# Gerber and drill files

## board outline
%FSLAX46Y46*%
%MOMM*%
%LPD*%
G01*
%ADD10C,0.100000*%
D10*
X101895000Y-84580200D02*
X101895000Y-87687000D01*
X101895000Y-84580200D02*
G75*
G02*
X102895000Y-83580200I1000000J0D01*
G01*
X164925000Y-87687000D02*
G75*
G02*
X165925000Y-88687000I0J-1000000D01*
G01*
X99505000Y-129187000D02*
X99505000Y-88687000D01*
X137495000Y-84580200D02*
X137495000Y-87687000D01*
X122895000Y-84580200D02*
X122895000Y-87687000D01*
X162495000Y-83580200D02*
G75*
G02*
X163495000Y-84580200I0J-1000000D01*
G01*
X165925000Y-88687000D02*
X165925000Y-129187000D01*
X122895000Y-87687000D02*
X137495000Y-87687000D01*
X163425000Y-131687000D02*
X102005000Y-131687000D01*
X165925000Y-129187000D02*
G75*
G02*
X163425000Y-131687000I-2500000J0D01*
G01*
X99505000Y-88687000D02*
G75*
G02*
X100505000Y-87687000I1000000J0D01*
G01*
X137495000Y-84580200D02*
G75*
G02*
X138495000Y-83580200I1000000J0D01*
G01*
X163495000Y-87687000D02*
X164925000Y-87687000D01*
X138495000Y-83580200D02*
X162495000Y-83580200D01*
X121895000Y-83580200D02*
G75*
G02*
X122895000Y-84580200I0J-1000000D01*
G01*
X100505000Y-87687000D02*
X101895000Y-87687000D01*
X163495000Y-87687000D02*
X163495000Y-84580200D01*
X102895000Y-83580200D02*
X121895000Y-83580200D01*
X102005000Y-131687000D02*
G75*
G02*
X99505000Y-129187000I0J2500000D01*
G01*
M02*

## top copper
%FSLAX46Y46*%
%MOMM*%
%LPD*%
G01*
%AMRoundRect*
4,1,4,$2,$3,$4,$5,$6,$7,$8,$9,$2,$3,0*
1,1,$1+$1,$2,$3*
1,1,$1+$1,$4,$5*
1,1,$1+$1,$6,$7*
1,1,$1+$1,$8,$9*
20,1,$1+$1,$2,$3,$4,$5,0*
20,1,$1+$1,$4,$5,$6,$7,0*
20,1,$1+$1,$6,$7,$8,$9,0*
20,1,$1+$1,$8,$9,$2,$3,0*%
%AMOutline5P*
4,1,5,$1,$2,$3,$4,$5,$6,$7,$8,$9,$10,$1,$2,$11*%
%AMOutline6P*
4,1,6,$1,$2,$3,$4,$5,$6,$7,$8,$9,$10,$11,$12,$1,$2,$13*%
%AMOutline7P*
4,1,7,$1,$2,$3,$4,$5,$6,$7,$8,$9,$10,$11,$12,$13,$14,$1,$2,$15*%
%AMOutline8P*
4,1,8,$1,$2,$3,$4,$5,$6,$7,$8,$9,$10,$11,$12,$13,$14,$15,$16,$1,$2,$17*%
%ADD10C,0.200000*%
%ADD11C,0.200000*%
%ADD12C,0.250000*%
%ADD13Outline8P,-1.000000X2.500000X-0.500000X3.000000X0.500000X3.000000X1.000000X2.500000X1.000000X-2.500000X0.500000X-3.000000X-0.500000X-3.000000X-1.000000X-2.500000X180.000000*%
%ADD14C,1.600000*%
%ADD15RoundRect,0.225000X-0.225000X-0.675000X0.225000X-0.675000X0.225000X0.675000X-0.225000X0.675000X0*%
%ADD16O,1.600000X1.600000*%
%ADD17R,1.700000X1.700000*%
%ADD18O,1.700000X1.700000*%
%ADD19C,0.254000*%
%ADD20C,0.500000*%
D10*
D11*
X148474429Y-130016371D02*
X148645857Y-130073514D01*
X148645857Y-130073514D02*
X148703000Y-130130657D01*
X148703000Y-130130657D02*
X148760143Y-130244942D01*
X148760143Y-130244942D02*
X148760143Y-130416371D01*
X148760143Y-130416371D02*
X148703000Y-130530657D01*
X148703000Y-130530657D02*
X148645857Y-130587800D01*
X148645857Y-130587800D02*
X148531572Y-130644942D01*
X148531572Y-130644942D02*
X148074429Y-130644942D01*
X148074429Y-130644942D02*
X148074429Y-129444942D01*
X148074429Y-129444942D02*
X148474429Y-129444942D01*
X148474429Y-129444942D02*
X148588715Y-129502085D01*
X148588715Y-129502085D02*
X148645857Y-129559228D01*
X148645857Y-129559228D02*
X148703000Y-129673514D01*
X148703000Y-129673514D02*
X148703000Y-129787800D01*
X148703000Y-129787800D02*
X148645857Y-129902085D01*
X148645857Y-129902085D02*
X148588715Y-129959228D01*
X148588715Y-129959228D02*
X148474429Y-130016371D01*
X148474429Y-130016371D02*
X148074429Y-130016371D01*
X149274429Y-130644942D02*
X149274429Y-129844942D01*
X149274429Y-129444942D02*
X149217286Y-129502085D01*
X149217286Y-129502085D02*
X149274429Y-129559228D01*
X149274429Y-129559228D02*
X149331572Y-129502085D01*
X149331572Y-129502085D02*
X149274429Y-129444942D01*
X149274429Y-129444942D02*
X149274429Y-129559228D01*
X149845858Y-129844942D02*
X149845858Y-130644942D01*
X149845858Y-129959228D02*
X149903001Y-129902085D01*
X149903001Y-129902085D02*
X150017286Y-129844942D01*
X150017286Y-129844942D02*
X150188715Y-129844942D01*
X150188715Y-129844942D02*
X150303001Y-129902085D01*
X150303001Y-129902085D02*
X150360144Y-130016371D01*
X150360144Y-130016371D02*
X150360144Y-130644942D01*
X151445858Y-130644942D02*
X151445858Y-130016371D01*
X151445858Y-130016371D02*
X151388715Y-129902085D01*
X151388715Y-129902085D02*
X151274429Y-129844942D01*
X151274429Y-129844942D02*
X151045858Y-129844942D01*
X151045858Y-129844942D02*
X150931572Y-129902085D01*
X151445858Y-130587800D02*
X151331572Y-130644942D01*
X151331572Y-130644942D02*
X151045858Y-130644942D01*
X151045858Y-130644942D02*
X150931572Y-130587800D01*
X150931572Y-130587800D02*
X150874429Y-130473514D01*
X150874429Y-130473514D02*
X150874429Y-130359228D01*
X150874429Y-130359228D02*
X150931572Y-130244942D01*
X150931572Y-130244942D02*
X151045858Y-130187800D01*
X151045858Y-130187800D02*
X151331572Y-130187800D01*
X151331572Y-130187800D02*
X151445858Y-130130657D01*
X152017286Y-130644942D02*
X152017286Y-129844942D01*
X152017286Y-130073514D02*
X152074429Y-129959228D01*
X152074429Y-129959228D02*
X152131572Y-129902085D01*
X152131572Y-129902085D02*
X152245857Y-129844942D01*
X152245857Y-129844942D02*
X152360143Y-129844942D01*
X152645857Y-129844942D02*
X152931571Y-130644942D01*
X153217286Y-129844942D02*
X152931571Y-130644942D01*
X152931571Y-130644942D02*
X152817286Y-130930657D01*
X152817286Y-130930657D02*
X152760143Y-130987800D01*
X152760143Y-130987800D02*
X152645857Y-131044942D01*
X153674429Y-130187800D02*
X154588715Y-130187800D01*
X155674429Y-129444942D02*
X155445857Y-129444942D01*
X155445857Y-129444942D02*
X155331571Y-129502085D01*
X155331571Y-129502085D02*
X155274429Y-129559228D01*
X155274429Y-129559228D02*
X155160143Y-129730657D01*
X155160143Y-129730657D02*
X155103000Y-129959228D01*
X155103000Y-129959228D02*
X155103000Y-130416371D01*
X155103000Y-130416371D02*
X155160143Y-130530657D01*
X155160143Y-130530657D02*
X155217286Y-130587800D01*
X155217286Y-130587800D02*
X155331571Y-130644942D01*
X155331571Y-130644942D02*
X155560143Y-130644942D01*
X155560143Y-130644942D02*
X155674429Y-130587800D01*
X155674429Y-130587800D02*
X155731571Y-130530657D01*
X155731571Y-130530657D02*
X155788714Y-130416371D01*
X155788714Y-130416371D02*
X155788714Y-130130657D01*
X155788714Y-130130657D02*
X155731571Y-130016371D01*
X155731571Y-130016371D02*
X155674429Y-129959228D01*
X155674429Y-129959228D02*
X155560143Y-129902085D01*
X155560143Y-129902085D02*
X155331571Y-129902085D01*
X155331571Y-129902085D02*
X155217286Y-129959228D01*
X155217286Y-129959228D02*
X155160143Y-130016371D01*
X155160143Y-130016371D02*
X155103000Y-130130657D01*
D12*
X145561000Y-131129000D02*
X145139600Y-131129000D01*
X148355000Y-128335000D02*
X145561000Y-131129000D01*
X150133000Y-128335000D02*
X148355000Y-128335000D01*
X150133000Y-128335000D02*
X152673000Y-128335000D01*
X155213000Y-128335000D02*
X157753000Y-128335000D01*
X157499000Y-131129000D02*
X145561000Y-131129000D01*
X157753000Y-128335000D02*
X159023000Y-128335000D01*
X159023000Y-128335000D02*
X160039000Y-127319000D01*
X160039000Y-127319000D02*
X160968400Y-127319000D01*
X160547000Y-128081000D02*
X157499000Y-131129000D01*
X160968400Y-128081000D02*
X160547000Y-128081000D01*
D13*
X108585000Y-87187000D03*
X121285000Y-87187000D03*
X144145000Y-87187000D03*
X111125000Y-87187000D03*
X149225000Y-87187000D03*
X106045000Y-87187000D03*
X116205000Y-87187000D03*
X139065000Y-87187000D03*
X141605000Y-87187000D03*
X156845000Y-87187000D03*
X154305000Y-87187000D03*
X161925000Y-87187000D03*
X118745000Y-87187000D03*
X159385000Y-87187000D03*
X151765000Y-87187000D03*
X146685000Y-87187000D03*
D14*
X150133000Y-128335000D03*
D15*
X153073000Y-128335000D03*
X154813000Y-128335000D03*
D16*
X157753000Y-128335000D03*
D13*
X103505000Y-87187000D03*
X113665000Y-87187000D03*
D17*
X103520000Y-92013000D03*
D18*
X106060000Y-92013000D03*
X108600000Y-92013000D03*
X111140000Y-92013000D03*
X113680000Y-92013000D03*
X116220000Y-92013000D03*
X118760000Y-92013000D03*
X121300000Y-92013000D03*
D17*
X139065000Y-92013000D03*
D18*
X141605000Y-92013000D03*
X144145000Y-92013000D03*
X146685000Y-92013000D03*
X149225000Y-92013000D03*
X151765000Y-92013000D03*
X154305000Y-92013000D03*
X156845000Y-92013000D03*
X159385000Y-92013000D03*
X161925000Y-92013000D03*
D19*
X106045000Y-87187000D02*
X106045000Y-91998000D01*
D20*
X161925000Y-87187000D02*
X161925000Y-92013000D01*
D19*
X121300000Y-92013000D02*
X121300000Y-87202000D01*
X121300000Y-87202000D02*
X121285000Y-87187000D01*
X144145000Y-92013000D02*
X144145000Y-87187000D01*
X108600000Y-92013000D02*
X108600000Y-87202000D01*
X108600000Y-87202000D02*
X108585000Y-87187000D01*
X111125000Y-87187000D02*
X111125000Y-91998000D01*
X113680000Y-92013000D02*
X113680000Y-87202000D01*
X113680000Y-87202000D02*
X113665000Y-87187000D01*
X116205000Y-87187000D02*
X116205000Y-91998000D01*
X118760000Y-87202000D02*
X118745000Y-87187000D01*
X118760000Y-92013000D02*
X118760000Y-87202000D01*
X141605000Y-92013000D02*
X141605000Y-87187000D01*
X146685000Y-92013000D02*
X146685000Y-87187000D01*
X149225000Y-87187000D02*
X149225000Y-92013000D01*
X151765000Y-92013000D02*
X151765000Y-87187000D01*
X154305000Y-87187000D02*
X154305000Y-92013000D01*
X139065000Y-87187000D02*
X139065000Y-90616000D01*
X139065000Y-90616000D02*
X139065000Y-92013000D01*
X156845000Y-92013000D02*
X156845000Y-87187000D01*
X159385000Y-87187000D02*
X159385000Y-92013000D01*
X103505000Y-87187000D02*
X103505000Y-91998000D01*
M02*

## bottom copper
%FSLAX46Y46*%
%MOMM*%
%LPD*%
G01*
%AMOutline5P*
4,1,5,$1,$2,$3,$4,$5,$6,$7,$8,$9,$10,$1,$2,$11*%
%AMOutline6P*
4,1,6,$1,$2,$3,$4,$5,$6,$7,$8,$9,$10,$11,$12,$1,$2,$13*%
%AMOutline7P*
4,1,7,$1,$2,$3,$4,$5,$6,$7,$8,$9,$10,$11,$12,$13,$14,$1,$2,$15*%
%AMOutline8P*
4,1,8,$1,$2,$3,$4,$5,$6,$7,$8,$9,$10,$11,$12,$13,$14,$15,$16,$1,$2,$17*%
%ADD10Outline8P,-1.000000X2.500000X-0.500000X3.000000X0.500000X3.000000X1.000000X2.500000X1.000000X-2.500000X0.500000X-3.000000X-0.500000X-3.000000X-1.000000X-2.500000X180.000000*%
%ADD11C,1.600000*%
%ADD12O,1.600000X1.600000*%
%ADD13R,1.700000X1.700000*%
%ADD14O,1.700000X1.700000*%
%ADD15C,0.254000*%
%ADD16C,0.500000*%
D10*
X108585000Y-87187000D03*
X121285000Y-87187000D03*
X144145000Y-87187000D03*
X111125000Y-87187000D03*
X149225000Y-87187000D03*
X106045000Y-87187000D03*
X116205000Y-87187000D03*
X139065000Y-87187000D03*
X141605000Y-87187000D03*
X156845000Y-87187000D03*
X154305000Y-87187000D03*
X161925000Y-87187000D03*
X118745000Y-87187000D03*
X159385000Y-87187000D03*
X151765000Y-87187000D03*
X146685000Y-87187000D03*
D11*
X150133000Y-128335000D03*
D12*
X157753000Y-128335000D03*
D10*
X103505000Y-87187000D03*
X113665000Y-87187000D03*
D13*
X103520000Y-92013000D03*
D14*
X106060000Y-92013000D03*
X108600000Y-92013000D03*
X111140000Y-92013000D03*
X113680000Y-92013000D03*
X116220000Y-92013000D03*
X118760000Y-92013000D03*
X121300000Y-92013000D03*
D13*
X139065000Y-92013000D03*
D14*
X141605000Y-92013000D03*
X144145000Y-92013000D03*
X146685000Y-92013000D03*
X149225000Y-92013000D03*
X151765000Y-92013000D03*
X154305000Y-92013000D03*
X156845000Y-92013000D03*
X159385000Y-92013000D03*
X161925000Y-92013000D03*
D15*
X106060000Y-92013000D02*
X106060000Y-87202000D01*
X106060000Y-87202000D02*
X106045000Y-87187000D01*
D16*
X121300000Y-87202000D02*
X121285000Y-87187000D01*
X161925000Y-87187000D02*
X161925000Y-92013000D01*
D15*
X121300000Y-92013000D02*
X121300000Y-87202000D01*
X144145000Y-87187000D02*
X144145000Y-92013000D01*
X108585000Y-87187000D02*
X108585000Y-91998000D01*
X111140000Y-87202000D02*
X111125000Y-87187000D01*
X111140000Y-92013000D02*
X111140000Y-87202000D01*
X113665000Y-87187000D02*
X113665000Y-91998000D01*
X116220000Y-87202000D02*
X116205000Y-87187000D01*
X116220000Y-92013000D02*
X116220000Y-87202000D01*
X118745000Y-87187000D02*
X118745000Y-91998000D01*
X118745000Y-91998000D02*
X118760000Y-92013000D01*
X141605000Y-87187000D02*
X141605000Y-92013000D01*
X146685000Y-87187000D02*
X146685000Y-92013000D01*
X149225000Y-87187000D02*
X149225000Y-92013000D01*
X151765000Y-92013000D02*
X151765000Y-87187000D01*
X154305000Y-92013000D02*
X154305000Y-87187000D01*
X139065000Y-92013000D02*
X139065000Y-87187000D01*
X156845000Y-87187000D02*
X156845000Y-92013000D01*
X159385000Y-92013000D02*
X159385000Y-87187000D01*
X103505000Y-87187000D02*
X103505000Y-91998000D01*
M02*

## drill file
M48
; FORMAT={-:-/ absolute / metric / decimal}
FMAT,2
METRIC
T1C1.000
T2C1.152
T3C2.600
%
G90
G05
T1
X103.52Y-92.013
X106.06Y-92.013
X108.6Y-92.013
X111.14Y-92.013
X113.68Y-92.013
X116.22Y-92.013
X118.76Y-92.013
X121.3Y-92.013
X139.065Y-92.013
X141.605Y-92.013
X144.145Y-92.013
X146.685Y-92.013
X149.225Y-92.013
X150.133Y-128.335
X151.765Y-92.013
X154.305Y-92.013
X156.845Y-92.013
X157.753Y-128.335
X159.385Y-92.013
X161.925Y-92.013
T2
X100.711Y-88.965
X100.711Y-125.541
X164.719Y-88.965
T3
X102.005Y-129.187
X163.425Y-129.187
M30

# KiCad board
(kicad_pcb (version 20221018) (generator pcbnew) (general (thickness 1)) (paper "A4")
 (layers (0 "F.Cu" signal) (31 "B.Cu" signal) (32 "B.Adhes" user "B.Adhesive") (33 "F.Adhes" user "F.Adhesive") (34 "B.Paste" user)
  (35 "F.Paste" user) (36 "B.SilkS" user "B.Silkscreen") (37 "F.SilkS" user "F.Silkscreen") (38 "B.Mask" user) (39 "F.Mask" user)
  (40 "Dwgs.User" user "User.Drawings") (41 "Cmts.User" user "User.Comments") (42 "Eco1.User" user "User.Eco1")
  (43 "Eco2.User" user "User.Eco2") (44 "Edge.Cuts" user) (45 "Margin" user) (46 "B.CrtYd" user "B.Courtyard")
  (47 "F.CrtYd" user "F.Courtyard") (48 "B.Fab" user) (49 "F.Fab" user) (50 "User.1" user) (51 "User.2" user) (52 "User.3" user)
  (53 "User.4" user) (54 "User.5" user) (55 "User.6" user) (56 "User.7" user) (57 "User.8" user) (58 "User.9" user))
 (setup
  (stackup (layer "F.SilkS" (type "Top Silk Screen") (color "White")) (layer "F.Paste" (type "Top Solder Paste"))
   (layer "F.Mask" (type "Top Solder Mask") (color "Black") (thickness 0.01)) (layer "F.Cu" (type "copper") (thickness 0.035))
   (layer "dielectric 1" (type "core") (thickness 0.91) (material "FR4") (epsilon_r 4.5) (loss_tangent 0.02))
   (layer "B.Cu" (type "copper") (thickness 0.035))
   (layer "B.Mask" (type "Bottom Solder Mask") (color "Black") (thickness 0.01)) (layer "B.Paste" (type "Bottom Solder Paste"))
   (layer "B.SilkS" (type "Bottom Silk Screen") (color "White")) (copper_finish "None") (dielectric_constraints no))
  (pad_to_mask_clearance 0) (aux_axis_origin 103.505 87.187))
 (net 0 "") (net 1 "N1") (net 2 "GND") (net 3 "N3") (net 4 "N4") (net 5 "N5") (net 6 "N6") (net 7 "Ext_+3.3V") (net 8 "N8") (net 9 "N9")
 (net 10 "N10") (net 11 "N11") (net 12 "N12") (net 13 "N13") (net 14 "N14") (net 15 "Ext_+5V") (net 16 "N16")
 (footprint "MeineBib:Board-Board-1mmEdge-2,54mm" (layer "F.Cu") (at 108.585 87.187)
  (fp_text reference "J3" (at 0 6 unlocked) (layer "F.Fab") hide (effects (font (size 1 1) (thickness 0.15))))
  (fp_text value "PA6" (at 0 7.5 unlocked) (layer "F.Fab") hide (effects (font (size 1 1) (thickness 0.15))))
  (pad "1" smd roundrect (at 0 0 180) (size 2 6) (layers "F.Cu" "F.Paste" "F.Mask") (roundrect_rratio 0) (chamfer_ratio 0.25)
   (chamfer top_left top_right bottom_left bottom_right) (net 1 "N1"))
  (pad "1" smd roundrect (at 0 0 180) (size 2 6) (layers "B.Cu" "B.Paste" "B.Mask") (roundrect_rratio 0) (chamfer_ratio 0.25)
   (chamfer top_left top_right bottom_left bottom_right) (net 1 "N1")))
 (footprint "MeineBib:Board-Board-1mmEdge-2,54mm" (layer "F.Cu") (at 121.285 87.187)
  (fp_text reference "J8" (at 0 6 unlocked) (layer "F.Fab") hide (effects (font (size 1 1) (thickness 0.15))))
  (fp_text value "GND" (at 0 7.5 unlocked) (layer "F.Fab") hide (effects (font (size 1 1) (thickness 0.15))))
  (pad "1" smd roundrect (at 0 0 180) (size 2 6) (layers "F.Cu" "F.Paste" "F.Mask") (roundrect_rratio 0) (chamfer_ratio 0.25)
   (chamfer top_left top_right bottom_left bottom_right) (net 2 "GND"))
  (pad "1" smd roundrect (at 0 0 180) (size 2 6) (layers "B.Cu" "B.Paste" "B.Mask") (roundrect_rratio 0) (chamfer_ratio 0.25)
   (chamfer top_left top_right bottom_left bottom_right) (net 2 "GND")))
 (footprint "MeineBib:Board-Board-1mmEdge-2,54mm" (layer "F.Cu") (at 144.145 87.187)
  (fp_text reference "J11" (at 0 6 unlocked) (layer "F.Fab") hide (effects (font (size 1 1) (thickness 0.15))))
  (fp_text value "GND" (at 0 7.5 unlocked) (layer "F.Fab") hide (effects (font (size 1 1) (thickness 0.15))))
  (pad "1" smd roundrect (at 0 0 180) (size 2 6) (layers "F.Cu" "F.Paste" "F.Mask") (roundrect_rratio 0) (chamfer_ratio 0.25)
   (chamfer top_left top_right bottom_left bottom_right) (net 2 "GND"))
  (pad "1" smd roundrect (at 0 0 180) (size 2 6) (layers "B.Cu" "B.Paste" "B.Mask") (roundrect_rratio 0) (chamfer_ratio 0.25)
   (chamfer top_left top_right bottom_left bottom_right) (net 2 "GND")))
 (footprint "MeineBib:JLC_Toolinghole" (layer "F.Cu") (at 164.719 88.965)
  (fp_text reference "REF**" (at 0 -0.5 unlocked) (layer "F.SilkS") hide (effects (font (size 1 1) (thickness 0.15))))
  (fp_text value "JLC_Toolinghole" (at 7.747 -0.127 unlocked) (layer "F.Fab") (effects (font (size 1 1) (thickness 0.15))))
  (pad "" np_thru_hole circle (at 0 0) (size 1.3 1.3) (drill 1.152) (layers "*.Mask")))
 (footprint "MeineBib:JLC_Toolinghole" (layer "F.Cu") (at 100.711 125.541)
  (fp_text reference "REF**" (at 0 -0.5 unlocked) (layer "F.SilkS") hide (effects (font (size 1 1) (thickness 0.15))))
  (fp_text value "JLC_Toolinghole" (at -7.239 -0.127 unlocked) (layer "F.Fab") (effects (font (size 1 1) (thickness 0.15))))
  (pad "" np_thru_hole circle (at 0 0) (size 1.3 1.3) (drill 1.152) (layers "*.Mask")))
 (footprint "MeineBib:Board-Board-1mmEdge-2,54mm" (layer "F.Cu") (at 111.125 87.187)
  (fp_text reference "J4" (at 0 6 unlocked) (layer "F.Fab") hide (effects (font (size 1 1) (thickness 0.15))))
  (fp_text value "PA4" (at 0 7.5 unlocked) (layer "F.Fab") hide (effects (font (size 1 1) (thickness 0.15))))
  (pad "1" smd roundrect (at 0 0 180) (size 2 6) (layers "F.Cu" "F.Paste" "F.Mask") (roundrect_rratio 0) (chamfer_ratio 0.25)
   (chamfer top_left top_right bottom_left bottom_right) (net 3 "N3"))
  (pad "1" smd roundrect (at 0 0 180) (size 2 6) (layers "B.Cu" "B.Paste" "B.Mask") (roundrect_rratio 0) (chamfer_ratio 0.25)
   (chamfer top_left top_right bottom_left bottom_right) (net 3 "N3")))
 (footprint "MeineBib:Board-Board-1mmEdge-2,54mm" (layer "F.Cu") (at 149.225 87.187)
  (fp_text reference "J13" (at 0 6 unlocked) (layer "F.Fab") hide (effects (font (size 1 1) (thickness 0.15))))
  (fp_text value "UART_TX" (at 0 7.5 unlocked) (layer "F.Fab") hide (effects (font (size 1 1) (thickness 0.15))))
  (pad "1" smd roundrect (at 0 0 180) (size 2 6) (layers "F.Cu" "F.Paste" "F.Mask") (roundrect_rratio 0) (chamfer_ratio 0.25)
   (chamfer top_left top_right bottom_left bottom_right) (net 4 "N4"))
  (pad "1" smd roundrect (at 0 0 180) (size 2 6) (layers "B.Cu" "B.Paste" "B.Mask") (roundrect_rratio 0) (chamfer_ratio 0.25)
   (chamfer top_left top_right bottom_left bottom_right) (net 4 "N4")))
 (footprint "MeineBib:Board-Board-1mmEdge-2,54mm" (layer "F.Cu") (at 106.045 87.187)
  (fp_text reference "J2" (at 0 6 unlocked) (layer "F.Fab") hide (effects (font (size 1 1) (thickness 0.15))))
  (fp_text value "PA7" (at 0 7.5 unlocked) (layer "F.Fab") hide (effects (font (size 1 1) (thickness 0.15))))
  (pad "1" smd roundrect (at 0 0 180) (size 2 6) (layers "F.Cu" "F.Paste" "F.Mask") (roundrect_rratio 0) (chamfer_ratio 0.25)
   (chamfer top_left top_right bottom_left bottom_right) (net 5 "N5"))
  (pad "1" smd roundrect (at 0 0 180) (size 2 6) (layers "B.Cu" "B.Paste" "B.Mask") (roundrect_rratio 0) (chamfer_ratio 0.25)
   (chamfer top_left top_right bottom_left bottom_right) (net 5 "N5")))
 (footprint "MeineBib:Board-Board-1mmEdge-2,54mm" (layer "F.Cu") (at 116.205 87.187)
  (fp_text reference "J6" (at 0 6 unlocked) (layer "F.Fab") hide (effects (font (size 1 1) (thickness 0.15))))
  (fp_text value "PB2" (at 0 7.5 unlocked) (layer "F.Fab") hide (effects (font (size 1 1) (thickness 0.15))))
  (pad "1" smd roundrect (at 0 0 180) (size 2 6) (layers "F.Cu" "F.Paste" "F.Mask") (roundrect_rratio 0) (chamfer_ratio 0.25)
   (chamfer top_left top_right bottom_left bottom_right) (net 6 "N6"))
  (pad "1" smd roundrect (at 0 0 180) (size 2 6) (layers "B.Cu" "B.Paste" "B.Mask") (roundrect_rratio 0) (chamfer_ratio 0.25)
   (chamfer top_left top_right bottom_left bottom_right) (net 6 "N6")))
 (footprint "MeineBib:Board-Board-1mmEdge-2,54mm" (layer "F.Cu") (at 139.065 87.187)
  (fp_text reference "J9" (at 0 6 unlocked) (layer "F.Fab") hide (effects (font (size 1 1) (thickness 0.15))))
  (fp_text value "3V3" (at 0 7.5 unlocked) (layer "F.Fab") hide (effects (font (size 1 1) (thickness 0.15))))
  (pad "1" smd roundrect (at 0 0 180) (size 2 6) (layers "F.Cu" "F.Paste" "F.Mask") (roundrect_rratio 0) (chamfer_ratio 0.25)
   (chamfer top_left top_right bottom_left bottom_right) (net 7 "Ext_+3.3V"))
  (pad "1" smd roundrect (at 0 0 180) (size 2 6) (layers "B.Cu" "B.Paste" "B.Mask") (roundrect_rratio 0) (chamfer_ratio 0.25)
   (chamfer top_left top_right bottom_left bottom_right) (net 7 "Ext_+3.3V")))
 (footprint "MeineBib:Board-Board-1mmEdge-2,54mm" (layer "F.Cu") (at 141.605 87.187)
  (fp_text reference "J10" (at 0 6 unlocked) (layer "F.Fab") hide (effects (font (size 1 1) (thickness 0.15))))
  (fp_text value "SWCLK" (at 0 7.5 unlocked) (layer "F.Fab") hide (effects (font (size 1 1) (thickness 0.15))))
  (pad "1" smd roundrect (at 0 0 180) (size 2 6) (layers "F.Cu" "F.Paste" "F.Mask") (roundrect_rratio 0) (chamfer_ratio 0.25)
   (chamfer top_left top_right bottom_left bottom_right) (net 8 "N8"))
  (pad "1" smd roundrect (at 0 0 180) (size 2 6) (layers "B.Cu" "B.Paste" "B.Mask") (roundrect_rratio 0) (chamfer_ratio 0.25)
   (chamfer top_left top_right bottom_left bottom_right) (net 8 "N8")))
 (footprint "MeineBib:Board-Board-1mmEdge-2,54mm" (layer "F.Cu") (at 156.845 87.187)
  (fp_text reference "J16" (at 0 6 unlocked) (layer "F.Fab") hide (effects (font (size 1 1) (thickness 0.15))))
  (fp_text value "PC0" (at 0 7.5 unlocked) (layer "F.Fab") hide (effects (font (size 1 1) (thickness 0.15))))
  (pad "1" smd roundrect (at 0 0 180) (size 2 6) (layers "F.Cu" "F.Paste" "F.Mask") (roundrect_rratio 0) (chamfer_ratio 0.25)
   (chamfer top_left top_right bottom_left bottom_right) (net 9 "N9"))
  (pad "1" smd roundrect (at 0 0 180) (size 2 6) (layers "B.Cu" "B.Paste" "B.Mask") (roundrect_rratio 0) (chamfer_ratio 0.25)
   (chamfer top_left top_right bottom_left bottom_right) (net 9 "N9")))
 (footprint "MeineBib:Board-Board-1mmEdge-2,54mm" (layer "F.Cu") (at 154.305 87.187)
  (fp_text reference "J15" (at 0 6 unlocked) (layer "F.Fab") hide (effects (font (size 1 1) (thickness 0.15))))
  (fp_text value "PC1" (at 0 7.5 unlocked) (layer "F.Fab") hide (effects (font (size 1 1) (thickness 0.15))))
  (pad "1" smd roundrect (at 0 0 180) (size 2 6) (layers "F.Cu" "F.Paste" "F.Mask") (roundrect_rratio 0) (chamfer_ratio 0.25)
   (chamfer top_left top_right bottom_left bottom_right) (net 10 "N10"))
  (pad "1" smd roundrect (at 0 0 180) (size 2 6) (layers "B.Cu" "B.Paste" "B.Mask") (roundrect_rratio 0) (chamfer_ratio 0.25)
   (chamfer top_left top_right bottom_left bottom_right) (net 10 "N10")))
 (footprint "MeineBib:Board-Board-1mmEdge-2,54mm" (layer "F.Cu") (at 161.925 87.187)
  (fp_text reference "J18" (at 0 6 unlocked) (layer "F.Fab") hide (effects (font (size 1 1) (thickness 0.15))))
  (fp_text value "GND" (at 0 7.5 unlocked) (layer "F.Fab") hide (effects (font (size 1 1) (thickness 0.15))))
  (pad "1" smd roundrect (at 0 0 180) (size 2 6) (layers "F.Cu" "F.Paste" "F.Mask") (roundrect_rratio 0) (chamfer_ratio 0.25)
   (chamfer top_left top_right bottom_left bottom_right) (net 2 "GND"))
  (pad "1" smd roundrect (at 0 0 180) (size 2 6) (layers "B.Cu" "B.Paste" "B.Mask") (roundrect_rratio 0) (chamfer_ratio 0.25)
   (chamfer top_left top_right bottom_left bottom_right) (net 2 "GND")))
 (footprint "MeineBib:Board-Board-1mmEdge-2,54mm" (layer "F.Cu") (at 118.745 87.187)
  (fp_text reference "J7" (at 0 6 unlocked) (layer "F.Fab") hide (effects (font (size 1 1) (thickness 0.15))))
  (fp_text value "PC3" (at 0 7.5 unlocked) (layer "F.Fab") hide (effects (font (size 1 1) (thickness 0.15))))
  (pad "1" smd roundrect (at 0 0 180) (size 2 6) (layers "F.Cu" "F.Paste" "F.Mask") (roundrect_rratio 0) (chamfer_ratio 0.25)
   (chamfer top_left top_right bottom_left bottom_right) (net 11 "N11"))
  (pad "1" smd roundrect (at 0 0 180) (size 2 6) (layers "B.Cu" "B.Paste" "B.Mask") (roundrect_rratio 0) (chamfer_ratio 0.25)
   (chamfer top_left top_right bottom_left bottom_right) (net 11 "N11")))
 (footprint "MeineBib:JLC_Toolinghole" (layer "F.Cu") (at 100.711 88.965)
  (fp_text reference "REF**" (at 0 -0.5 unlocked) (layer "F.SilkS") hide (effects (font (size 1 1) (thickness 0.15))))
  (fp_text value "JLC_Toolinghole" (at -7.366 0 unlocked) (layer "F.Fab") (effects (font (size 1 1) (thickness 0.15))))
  (pad "" np_thru_hole circle (at 0 0) (size 1.3 1.3) (drill 1.152) (layers "*.Mask")))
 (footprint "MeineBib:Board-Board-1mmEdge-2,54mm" (layer "F.Cu") (at 159.385 87.187)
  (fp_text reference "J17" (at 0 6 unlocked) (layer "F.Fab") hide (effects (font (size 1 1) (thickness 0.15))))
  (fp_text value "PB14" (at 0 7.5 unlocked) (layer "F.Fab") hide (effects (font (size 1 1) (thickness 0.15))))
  (pad "1" smd roundrect (at 0 0 180) (size 2 6) (layers "F.Cu" "F.Paste" "F.Mask") (roundrect_rratio 0) (chamfer_ratio 0.25)
   (chamfer top_left top_right bottom_left bottom_right) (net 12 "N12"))
  (pad "1" smd roundrect (at 0 0 180) (size 2 6) (layers "B.Cu" "B.Paste" "B.Mask") (roundrect_rratio 0) (chamfer_ratio 0.25)
   (chamfer top_left top_right bottom_left bottom_right) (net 12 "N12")))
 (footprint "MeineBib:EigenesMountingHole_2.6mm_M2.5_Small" (layer "F.Cu") (at 102.005 129.187)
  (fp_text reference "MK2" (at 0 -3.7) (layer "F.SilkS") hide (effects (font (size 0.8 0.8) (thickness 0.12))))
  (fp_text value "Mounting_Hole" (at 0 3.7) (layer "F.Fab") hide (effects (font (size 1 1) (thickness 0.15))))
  (pad "" np_thru_hole circle (at 0 0) (size 2.6 2.6) (drill 2.6) (layers "F&B.Cu" "*.Mask") (solder_mask_margin 1.25) (clearance 1.25)))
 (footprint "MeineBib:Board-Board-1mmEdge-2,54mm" (layer "F.Cu") (at 151.765 87.187)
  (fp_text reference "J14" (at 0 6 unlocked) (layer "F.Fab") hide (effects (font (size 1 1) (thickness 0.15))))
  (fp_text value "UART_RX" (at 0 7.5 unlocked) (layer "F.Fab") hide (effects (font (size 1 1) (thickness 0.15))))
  (pad "1" smd roundrect (at 0 0 180) (size 2 6) (layers "F.Cu" "F.Paste" "F.Mask") (roundrect_rratio 0) (chamfer_ratio 0.25)
   (chamfer top_left top_right bottom_left bottom_right) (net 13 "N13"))
  (pad "1" smd roundrect (at 0 0 180) (size 2 6) (layers "B.Cu" "B.Paste" "B.Mask") (roundrect_rratio 0) (chamfer_ratio 0.25)
   (chamfer top_left top_right bottom_left bottom_right) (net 13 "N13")))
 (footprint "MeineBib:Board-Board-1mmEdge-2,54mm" (layer "F.Cu") (at 146.685 87.187)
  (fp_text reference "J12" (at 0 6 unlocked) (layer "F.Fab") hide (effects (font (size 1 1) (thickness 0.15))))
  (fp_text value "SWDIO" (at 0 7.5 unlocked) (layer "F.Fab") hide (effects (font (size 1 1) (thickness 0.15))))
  (pad "1" smd roundrect (at 0 0 180) (size 2 6) (layers "F.Cu" "F.Paste" "F.Mask") (roundrect_rratio 0) (chamfer_ratio 0.25)
   (chamfer top_left top_right bottom_left bottom_right) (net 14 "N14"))
  (pad "1" smd roundrect (at 0 0 180) (size 2 6) (layers "B.Cu" "B.Paste" "B.Mask") (roundrect_rratio 0) (chamfer_ratio 0.25)
   (chamfer top_left top_right bottom_left bottom_right) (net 14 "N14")))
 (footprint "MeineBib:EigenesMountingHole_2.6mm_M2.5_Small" (layer "F.Cu") (at 163.425 129.187)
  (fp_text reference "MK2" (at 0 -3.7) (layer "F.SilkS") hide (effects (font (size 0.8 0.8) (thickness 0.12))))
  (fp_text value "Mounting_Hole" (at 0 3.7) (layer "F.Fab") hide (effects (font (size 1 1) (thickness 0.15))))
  (pad "" np_thru_hole circle (at 0 0) (size 2.6 2.6) (drill 2.6) (layers "F&B.Cu" "*.Mask") (solder_mask_margin 1.25) (clearance 1.25)))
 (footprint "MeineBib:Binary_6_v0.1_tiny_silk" (layer "F.Cu") (at 153.9684 129.3002) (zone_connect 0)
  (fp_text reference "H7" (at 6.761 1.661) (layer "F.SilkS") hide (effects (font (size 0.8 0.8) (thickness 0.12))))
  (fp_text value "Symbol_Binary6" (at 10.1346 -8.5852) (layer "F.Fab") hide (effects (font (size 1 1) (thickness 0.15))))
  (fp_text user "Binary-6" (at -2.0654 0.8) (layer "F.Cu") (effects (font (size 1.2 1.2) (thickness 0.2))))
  (fp_line (start -8.4074 1.8288) (end -8.8288 1.8288) (stroke (width 0.25) (type solid)) (layer "F.Cu"))
  (fp_line (start -5.6134 -0.9652) (end -8.4074 1.8288) (stroke (width 0.25) (type solid)) (layer "F.Cu"))
  (fp_line (start -3.8354 -0.9652) (end -5.6134 -0.9652) (stroke (width 0.25) (type solid)) (layer "F.Cu"))
  (fp_line (start -3.8354 -0.9652) (end -1.2954 -0.9652) (stroke (width 0.25) (type solid)) (layer "F.Cu"))
  (fp_line (start 1.2446 -0.9652) (end 3.7846 -0.9652) (stroke (width 0.25) (type solid)) (layer "F.Cu"))
  (fp_line (start 3.5306 1.8288) (end -8.4074 1.8288) (stroke (width 0.25) (type solid)) (layer "F.Cu"))
  (fp_line (start 3.7846 -0.9652) (end 5.0546 -0.9652) (stroke (width 0.25) (type solid)) (layer "F.Cu"))
  (fp_line (start 5.0546 -0.9652) (end 6.0706 -1.9812) (stroke (width 0.25) (type solid)) (layer "F.Cu"))
  (fp_line (start 6.0706 -1.9812) (end 7 -1.9812) (stroke (width 0.25) (type solid)) (layer "F.Cu"))
  (fp_line (start 6.5786 -1.2192) (end 3.5306 1.8288) (stroke (width 0.25) (type solid)) (layer "F.Cu"))
  (fp_line (start 7 -1.2192) (end 6.5786 -1.2192) (stroke (width 0.25) (type solid)) (layer "F.Cu"))
  (pad "" thru_hole circle (at -3.8354 -0.9652) (size 1.6 1.6) (drill 1) (layers "*.Cu" "*.Mask") (zone_connect 0))
  (pad "" smd roundrect (at -0.8954 -0.9652) (size 0.9 1.8) (layers "F.Cu" "F.Mask") (roundrect_rratio 0.25) (zone_connect 0))
  (pad "" smd roundrect (at 0.8446 -0.9652) (size 0.9 1.8) (layers "F.Cu" "F.Mask") (roundrect_rratio 0.25) (zone_connect 0))
  (pad "" thru_hole oval (at 3.7846 -0.9652) (size 1.6 1.6) (drill 1) (layers "*.Cu" "*.Mask") (zone_connect 0)))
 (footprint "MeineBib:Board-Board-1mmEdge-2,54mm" (layer "F.Cu") (at 103.505 87.187)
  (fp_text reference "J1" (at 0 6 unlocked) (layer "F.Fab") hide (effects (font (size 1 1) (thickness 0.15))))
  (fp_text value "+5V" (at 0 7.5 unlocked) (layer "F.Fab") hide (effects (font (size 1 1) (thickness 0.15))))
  (pad "1" smd roundrect (at 0 0 180) (size 2 6) (layers "F.Cu" "F.Paste" "F.Mask") (roundrect_rratio 0) (chamfer_ratio 0.25)
   (chamfer top_left top_right bottom_left bottom_right) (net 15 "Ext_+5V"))
  (pad "1" smd roundrect (at 0 0 180) (size 2 6) (layers "B.Cu" "B.Paste" "B.Mask") (roundrect_rratio 0) (chamfer_ratio 0.25)
   (chamfer top_left top_right bottom_left bottom_right) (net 15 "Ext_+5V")))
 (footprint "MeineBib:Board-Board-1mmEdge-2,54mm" (layer "F.Cu") (at 113.665 87.187)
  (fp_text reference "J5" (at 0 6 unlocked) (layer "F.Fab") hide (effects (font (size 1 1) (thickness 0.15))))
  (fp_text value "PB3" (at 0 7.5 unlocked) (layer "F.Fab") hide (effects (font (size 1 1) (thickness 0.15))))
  (pad "1" smd roundrect (at 0 0 180) (size 2 6) (layers "F.Cu" "F.Paste" "F.Mask") (roundrect_rratio 0) (chamfer_ratio 0.25)
   (chamfer top_left top_right bottom_left bottom_right) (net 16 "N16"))
  (pad "1" smd roundrect (at 0 0 180) (size 2 6) (layers "B.Cu" "B.Paste" "B.Mask") (roundrect_rratio 0) (chamfer_ratio 0.25)
   (chamfer top_left top_right bottom_left bottom_right) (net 16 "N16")))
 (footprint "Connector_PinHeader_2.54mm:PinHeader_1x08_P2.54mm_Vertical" (layer "B.Cu") (at 103.52 92.013 -90)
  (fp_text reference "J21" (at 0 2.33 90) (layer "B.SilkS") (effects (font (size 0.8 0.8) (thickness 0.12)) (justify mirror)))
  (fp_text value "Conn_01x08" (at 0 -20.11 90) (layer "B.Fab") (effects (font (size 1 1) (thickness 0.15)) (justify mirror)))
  (pad "1" thru_hole rect (at 0 0 270) (size 1.7 1.7) (drill 1) (layers "*.Cu" "*.Mask") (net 15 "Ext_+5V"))
  (pad "2" thru_hole oval (at 0 -2.54 270) (size 1.7 1.7) (drill 1) (layers "*.Cu" "*.Mask") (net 5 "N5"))
  (pad "3" thru_hole oval (at 0 -5.08 270) (size 1.7 1.7) (drill 1) (layers "*.Cu" "*.Mask") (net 1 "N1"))
  (pad "4" thru_hole oval (at 0 -7.62 270) (size 1.7 1.7) (drill 1) (layers "*.Cu" "*.Mask") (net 3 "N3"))
  (pad "5" thru_hole oval (at 0 -10.16 270) (size 1.7 1.7) (drill 1) (layers "*.Cu" "*.Mask") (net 16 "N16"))
  (pad "6" thru_hole oval (at 0 -12.7 270) (size 1.7 1.7) (drill 1) (layers "*.Cu" "*.Mask") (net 6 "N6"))
  (pad "7" thru_hole oval (at 0 -15.24 270) (size 1.7 1.7) (drill 1) (layers "*.Cu" "*.Mask") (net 11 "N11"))
  (pad "8" thru_hole oval (at 0 -17.78 270) (size 1.7 1.7) (drill 1) (layers "*.Cu" "*.Mask") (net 2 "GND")))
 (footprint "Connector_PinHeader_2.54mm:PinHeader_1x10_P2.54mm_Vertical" (layer "B.Cu") (at 139.065 92.013 -90)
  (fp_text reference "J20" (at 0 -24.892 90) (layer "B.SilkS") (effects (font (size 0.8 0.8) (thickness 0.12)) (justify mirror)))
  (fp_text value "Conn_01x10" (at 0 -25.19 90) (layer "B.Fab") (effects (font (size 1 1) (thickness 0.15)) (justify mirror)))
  (pad "1" thru_hole rect (at 0 0 270) (size 1.7 1.7) (drill 1) (layers "*.Cu" "*.Mask") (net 7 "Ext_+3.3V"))
  (pad "2" thru_hole oval (at 0 -2.54 270) (size 1.7 1.7) (drill 1) (layers "*.Cu" "*.Mask") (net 8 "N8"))
  (pad "3" thru_hole oval (at 0 -5.08 270) (size 1.7 1.7) (drill 1) (layers "*.Cu" "*.Mask") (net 2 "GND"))
  (pad "4" thru_hole oval (at 0 -7.62 270) (size 1.7 1.7) (drill 1) (layers "*.Cu" "*.Mask") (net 14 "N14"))
  (pad "5" thru_hole oval (at 0 -10.16 270) (size 1.7 1.7) (drill 1) (layers "*.Cu" "*.Mask") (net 4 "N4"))
  (pad "6" thru_hole oval (at 0 -12.7 270) (size 1.7 1.7) (drill 1) (layers "*.Cu" "*.Mask") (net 13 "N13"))
  (pad "7" thru_hole oval (at 0 -15.24 270) (size 1.7 1.7) (drill 1) (layers "*.Cu" "*.Mask") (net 10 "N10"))
  (pad "8" thru_hole oval (at 0 -17.78 270) (size 1.7 1.7) (drill 1) (layers "*.Cu" "*.Mask") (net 9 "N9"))
  (pad "9" thru_hole oval (at 0 -20.32 270) (size 1.7 1.7) (drill 1) (layers "*.Cu" "*.Mask") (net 12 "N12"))
  (pad "10" thru_hole oval (at 0 -22.86 270) (size 1.7 1.7) (drill 1) (layers "*.Cu" "*.Mask") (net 2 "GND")))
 (gr_line (start 101.895 84.5802) (end 101.895 87.687) (stroke (width 0.1) (type solid)) (layer "Edge.Cuts"))
 (gr_arc (start 101.895 84.5802) (mid 102.187893 83.873093) (end 102.895 83.5802) (stroke (width 0.1) (type solid)) (layer "Edge.Cuts"))
 (gr_arc (start 164.925 87.687) (mid 165.632107 87.979893) (end 165.925 88.687) (stroke (width 0.1) (type solid)) (layer "Edge.Cuts"))
 (gr_line (start 99.505 129.187) (end 99.505 88.687) (stroke (width 0.1) (type solid)) (layer "Edge.Cuts"))
 (gr_line (start 137.495 84.5802) (end 137.495 87.687) (stroke (width 0.1) (type solid)) (layer "Edge.Cuts"))
 (gr_line (start 122.895 84.5802) (end 122.895 87.687) (stroke (width 0.1) (type solid)) (layer "Edge.Cuts"))
 (gr_arc (start 162.495 83.5802) (mid 163.202107 83.873093) (end 163.495 84.5802) (stroke (width 0.1) (type solid)) (layer "Edge.Cuts"))
 (gr_line (start 165.925 88.687) (end 165.925 129.187) (stroke (width 0.1) (type solid)) (layer "Edge.Cuts"))
 (gr_line (start 122.895 87.687) (end 137.495 87.687) (stroke (width 0.1) (type solid)) (layer "Edge.Cuts"))
 (gr_line (start 163.425 131.687) (end 102.005 131.687) (stroke (width 0.1) (type solid)) (layer "Edge.Cuts"))
 (gr_arc (start 165.925 129.187) (mid 165.192767 130.954767) (end 163.425 131.687) (stroke (width 0.1) (type solid)) (layer "Edge.Cuts"))
 (gr_arc (start 99.505 88.687) (mid 99.797893 87.979893) (end 100.505 87.687) (stroke (width 0.1) (type solid)) (layer "Edge.Cuts"))
 (gr_arc (start 137.495 84.5802) (mid 137.787893 83.873093) (end 138.495 83.5802) (stroke (width 0.1) (type solid)) (layer "Edge.Cuts"))
 (gr_line (start 163.495 87.687) (end 164.925 87.687) (stroke (width 0.1) (type solid)) (layer "Edge.Cuts"))
 (gr_line (start 138.495 83.5802) (end 162.495 83.5802) (stroke (width 0.1) (type solid)) (layer "Edge.Cuts"))
 (gr_arc (start 121.895 83.5802) (mid 122.602107 83.873093) (end 122.895 84.5802) (stroke (width 0.1) (type solid)) (layer "Edge.Cuts"))
 (gr_line (start 100.505 87.687) (end 101.895 87.687) (stroke (width 0.1) (type solid)) (layer "Edge.Cuts"))
 (gr_line (start 163.495 87.687) (end 163.495 84.5802) (stroke (width 0.1) (type solid)) (layer "Edge.Cuts"))
 (gr_line (start 102.895 83.5802) (end 121.895 83.5802) (stroke (width 0.1) (type solid)) (layer "Edge.Cuts"))
 (gr_arc (start 102.005 131.687) (mid 100.237233 130.954767) (end 99.505 129.187) (stroke (width 0.1) (type solid)) (layer "Edge.Cuts"))
 (segment (start 106.045 87.187) (end 106.045 91.998) (width 0.254) (layer "F.Cu") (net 5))
 (segment (start 106.06 92.013) (end 106.06 87.202) (width 0.254) (layer "B.Cu") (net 5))
 (segment (start 106.06 87.202) (end 106.045 87.187) (width 0.254) (layer "B.Cu") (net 5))
 (segment (start 161.925 87.187) (end 161.925 92.013) (width 0.5) (layer "F.Cu") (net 2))
 (segment (start 121.3 92.013) (end 121.3 87.202) (width 0.254) (layer "F.Cu") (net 2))
 (segment (start 121.3 87.202) (end 121.285 87.187) (width 0.254) (layer "F.Cu") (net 2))
 (segment (start 144.145 92.013) (end 144.145 87.187) (width 0.254) (layer "F.Cu") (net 2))
 (segment (start 121.3 87.202) (end 121.285 87.187) (width 0.5) (layer "B.Cu") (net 2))
 (segment (start 161.925 87.187) (end 161.925 92.013) (width 0.5) (layer "B.Cu") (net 2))
 (segment (start 121.3 92.013) (end 121.3 87.202) (width 0.254) (layer "B.Cu") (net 2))
 (segment (start 144.145 87.187) (end 144.145 92.013) (width 0.254) (layer "B.Cu") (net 2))
 (segment (start 108.6 92.013) (end 108.6 87.202) (width 0.254) (layer "F.Cu") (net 1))
 (segment (start 108.6 87.202) (end 108.585 87.187) (width 0.254) (layer "F.Cu") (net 1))
 (segment (start 108.585 87.187) (end 108.585 91.998) (width 0.254) (layer "B.Cu") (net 1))
 (segment (start 111.125 87.187) (end 111.125 91.998) (width 0.254) (layer "F.Cu") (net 3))
 (segment (start 111.14 87.202) (end 111.125 87.187) (width 0.254) (layer "B.Cu") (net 3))
 (segment (start 111.14 92.013) (end 111.14 87.202) (width 0.254) (layer "B.Cu") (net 3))
 (segment (start 113.68 92.013) (end 113.68 87.202) (width 0.254) (layer "F.Cu") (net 16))
 (segment (start 113.68 87.202) (end 113.665 87.187) (width 0.254) (layer "F.Cu") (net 16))
 (segment (start 113.665 87.187) (end 113.665 91.998) (width 0.254) (layer "B.Cu") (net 16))
 (segment (start 116.205 87.187) (end 116.205 91.998) (width 0.254) (layer "F.Cu") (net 6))
 (segment (start 116.22 87.202) (end 116.205 87.187) (width 0.254) (layer "B.Cu") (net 6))
 (segment (start 116.22 92.013) (end 116.22 87.202) (width 0.254) (layer "B.Cu") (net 6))
 (segment (start 118.76 87.202) (end 118.745 87.187) (width 0.254) (layer "F.Cu") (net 11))
 (segment (start 118.76 92.013) (end 118.76 87.202) (width 0.254) (layer "F.Cu") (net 11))
 (segment (start 118.745 87.187) (end 118.745 91.998) (width 0.254) (layer "B.Cu") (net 11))
 (segment (start 118.745 91.998) (end 118.76 92.013) (width 0.254) (layer "B.Cu") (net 11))
 (segment (start 141.605 92.013) (end 141.605 87.187) (width 0.254) (layer "F.Cu") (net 8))
 (segment (start 141.605 87.187) (end 141.605 92.013) (width 0.254) (layer "B.Cu") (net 8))
 (segment (start 146.685 92.013) (end 146.685 87.187) (width 0.254) (layer "F.Cu") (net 14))
 (segment (start 146.685 87.187) (end 146.685 92.013) (width 0.254) (layer "B.Cu") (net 14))
 (segment (start 149.225 87.187) (end 149.225 92.013) (width 0.254) (layer "F.Cu") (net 4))
 (segment (start 149.225 87.187) (end 149.225 92.013) (width 0.254) (layer "B.Cu") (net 4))
 (segment (start 151.765 92.013) (end 151.765 87.187) (width 0.254) (layer "F.Cu") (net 13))
 (segment (start 151.765 92.013) (end 151.765 87.187) (width 0.254) (layer "B.Cu") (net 13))
 (segment (start 154.305 87.187) (end 154.305 92.013) (width 0.254) (layer "F.Cu") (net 10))
 (segment (start 154.305 92.013) (end 154.305 87.187) (width 0.254) (layer "B.Cu") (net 10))
 (segment (start 139.065 87.187) (end 139.065 90.616) (width 0.254) (layer "F.Cu") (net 7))
 (segment (start 139.065 90.616) (end 139.065 92.013) (width 0.254) (layer "F.Cu") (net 7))
 (segment (start 139.065 92.013) (end 139.065 87.187) (width 0.254) (layer "B.Cu") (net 7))
 (segment (start 156.845 92.013) (end 156.845 87.187) (width 0.254) (layer "F.Cu") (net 9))
 (segment (start 156.845 87.187) (end 156.845 92.013) (width 0.254) (layer "B.Cu") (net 9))
 (segment (start 159.385 87.187) (end 159.385 92.013) (width 0.254) (layer "F.Cu") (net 12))
 (segment (start 159.385 92.013) (end 159.385 87.187) (width 0.254) (layer "B.Cu") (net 12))
 (segment (start 103.505 87.187) (end 103.505 91.998) (width 0.254) (layer "F.Cu") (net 15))
 (segment (start 103.505 87.187) (end 103.505 91.998) (width 0.254) (layer "B.Cu") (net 15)))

